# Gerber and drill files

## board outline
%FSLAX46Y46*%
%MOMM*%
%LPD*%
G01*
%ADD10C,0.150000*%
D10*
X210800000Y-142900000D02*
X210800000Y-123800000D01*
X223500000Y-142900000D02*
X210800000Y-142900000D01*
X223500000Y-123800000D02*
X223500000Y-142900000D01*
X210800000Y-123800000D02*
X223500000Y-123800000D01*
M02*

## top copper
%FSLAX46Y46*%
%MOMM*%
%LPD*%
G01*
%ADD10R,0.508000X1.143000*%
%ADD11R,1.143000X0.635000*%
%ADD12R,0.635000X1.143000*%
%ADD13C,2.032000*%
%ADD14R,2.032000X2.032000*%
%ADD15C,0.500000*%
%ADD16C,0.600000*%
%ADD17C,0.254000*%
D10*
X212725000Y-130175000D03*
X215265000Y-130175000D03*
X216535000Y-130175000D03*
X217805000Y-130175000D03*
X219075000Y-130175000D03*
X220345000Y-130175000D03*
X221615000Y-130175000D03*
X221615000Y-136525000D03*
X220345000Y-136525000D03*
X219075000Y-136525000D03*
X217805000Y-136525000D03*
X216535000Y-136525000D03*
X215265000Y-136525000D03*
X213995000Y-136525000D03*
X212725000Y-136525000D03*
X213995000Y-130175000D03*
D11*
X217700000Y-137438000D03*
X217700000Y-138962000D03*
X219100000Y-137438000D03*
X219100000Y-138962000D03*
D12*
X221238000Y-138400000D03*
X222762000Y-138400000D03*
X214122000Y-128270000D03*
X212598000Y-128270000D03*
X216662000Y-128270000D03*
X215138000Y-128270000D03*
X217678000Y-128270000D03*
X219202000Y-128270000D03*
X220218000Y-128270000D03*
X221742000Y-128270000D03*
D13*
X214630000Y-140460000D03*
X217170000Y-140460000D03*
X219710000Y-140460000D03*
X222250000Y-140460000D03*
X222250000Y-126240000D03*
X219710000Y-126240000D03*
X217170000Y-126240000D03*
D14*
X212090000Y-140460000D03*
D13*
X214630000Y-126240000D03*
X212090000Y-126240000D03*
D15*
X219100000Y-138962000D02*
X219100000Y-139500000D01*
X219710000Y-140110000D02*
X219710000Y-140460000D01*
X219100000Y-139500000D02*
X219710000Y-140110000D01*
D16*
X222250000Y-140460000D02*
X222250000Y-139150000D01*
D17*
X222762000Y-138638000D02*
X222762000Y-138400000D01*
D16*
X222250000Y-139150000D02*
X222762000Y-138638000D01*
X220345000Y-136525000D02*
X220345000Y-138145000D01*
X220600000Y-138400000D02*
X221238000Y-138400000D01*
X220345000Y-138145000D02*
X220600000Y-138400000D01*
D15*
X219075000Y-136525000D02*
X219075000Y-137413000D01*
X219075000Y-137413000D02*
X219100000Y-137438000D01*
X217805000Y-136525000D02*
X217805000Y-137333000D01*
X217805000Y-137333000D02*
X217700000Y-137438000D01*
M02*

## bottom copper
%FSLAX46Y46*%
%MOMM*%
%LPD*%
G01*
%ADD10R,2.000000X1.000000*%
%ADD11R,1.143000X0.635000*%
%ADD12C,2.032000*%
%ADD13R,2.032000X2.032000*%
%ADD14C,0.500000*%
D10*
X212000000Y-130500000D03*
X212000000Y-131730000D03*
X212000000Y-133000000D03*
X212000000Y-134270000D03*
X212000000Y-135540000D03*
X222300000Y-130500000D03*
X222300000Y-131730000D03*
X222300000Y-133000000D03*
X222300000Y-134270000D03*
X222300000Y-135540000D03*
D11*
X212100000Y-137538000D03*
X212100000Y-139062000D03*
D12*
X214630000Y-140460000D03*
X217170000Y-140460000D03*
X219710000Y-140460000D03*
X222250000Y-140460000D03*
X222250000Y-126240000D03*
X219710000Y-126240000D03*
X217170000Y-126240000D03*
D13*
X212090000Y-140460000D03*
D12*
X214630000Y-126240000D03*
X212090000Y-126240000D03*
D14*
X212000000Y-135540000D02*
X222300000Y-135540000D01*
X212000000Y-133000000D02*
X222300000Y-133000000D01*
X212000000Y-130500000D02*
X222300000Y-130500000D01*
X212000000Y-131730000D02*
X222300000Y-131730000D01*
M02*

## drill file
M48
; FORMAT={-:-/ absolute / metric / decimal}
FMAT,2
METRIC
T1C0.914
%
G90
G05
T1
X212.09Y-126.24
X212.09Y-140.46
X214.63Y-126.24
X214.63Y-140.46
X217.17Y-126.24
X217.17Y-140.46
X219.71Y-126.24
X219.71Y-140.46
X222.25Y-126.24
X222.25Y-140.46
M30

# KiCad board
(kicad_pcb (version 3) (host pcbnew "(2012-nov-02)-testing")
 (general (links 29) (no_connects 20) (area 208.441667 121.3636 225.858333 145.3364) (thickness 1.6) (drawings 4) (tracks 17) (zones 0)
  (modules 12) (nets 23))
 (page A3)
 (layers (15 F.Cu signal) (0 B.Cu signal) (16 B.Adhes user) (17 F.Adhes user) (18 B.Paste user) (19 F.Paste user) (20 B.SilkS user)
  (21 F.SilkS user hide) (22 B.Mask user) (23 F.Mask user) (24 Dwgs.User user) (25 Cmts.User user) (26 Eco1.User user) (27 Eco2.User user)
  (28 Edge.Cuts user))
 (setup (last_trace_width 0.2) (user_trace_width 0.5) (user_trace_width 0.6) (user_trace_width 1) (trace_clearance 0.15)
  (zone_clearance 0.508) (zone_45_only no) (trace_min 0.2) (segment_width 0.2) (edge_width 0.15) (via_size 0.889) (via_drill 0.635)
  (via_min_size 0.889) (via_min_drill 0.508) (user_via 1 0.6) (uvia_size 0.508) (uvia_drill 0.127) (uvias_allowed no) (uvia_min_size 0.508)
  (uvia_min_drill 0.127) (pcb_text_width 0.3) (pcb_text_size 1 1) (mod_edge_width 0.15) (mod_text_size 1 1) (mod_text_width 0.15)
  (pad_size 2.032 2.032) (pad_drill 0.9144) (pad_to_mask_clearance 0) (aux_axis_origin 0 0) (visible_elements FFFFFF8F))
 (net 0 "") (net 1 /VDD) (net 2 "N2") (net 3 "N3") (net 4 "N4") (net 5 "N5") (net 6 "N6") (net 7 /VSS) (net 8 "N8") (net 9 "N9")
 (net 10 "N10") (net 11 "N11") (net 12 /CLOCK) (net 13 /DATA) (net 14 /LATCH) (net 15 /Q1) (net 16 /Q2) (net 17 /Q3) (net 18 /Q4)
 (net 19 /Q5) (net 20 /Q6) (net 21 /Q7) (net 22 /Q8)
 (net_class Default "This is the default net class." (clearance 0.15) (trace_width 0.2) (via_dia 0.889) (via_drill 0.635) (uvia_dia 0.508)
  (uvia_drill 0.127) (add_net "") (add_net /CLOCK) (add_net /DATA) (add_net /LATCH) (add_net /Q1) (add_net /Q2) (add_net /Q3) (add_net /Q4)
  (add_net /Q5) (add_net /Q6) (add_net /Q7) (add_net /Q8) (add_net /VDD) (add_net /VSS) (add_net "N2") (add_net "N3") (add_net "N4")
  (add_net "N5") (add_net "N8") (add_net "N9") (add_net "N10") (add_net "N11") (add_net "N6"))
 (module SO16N (layer F.Cu) (at 217.17 133.35)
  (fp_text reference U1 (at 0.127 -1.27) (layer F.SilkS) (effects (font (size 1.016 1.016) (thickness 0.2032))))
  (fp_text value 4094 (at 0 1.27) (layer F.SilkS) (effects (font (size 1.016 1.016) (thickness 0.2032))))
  (pad 16 smd rect (at -4.445 -3.175) (size 0.508 1.143) (layers F.Cu F.Paste F.Mask) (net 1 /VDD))
  (pad 14 smd rect (at -1.905 -3.175) (size 0.508 1.143) (layers F.Cu F.Paste F.Mask) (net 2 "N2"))
  (pad 13 smd rect (at -0.635 -3.175) (size 0.508 1.143) (layers F.Cu F.Paste F.Mask) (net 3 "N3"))
  (pad 12 smd rect (at 0.635 -3.175) (size 0.508 1.143) (layers F.Cu F.Paste F.Mask) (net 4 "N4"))
  (pad 11 smd rect (at 1.905 -3.175) (size 0.508 1.143) (layers F.Cu F.Paste F.Mask) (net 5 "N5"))
  (pad 10 smd rect (at 3.175 -3.175) (size 0.508 1.143) (layers F.Cu F.Paste F.Mask) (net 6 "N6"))
  (pad 9 smd rect (at 4.445 -3.175) (size 0.508 1.143) (layers F.Cu F.Paste F.Mask))
  (pad 8 smd rect (at 4.445 3.175) (size 0.508 1.143) (layers F.Cu F.Paste F.Mask) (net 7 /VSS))
  (pad 7 smd rect (at 3.175 3.175) (size 0.508 1.143) (layers F.Cu F.Paste F.Mask) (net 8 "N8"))
  (pad 6 smd rect (at 1.905 3.175) (size 0.508 1.143) (layers F.Cu F.Paste F.Mask) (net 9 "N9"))
  (pad 5 smd rect (at 0.635 3.175) (size 0.508 1.143) (layers F.Cu F.Paste F.Mask) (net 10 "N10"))
  (pad 4 smd rect (at -0.635 3.175) (size 0.508 1.143) (layers F.Cu F.Paste F.Mask) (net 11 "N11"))
  (pad 3 smd rect (at -1.905 3.175) (size 0.508 1.143) (layers F.Cu F.Paste F.Mask) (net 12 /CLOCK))
  (pad 2 smd rect (at -3.175 3.175) (size 0.508 1.143) (layers F.Cu F.Paste F.Mask) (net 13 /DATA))
  (pad 1 smd rect (at -4.445 3.175) (size 0.508 1.143) (layers F.Cu F.Paste F.Mask) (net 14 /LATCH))
  (pad 15 smd rect (at -3.175 -3.175) (size 0.508 1.143) (layers F.Cu F.Paste F.Mask) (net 1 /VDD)))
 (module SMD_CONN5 (layer B.Cu) (at 212 133 180)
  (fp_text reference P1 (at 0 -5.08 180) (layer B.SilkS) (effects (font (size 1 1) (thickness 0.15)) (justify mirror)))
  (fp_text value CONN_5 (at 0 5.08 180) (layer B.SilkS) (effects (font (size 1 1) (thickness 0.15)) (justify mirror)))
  (pad 1 smd rect (at 0 2.5 180) (size 2 1) (layers B.Cu B.Paste B.Mask) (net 1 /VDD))
  (pad 2 smd rect (at 0 1.27 180) (size 2 1) (layers B.Cu B.Paste B.Mask) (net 7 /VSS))
  (pad 3 smd rect (at 0 0 180) (size 2 1) (layers B.Cu B.Paste B.Mask) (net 14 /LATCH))
  (pad 4 smd rect (at 0 -1.27 180) (size 2 1) (layers B.Cu B.Paste B.Mask) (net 13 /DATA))
  (pad 5 smd rect (at 0 -2.54 180) (size 2 1) (layers B.Cu B.Paste B.Mask) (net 12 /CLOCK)))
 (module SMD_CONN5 (layer B.Cu) (at 222.3 133 180)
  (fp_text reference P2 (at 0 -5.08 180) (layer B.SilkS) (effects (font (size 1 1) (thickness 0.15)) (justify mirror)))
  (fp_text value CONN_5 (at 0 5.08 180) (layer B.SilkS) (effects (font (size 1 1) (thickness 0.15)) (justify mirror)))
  (pad 1 smd rect (at 0 2.5 180) (size 2 1) (layers B.Cu B.Paste B.Mask) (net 1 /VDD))
  (pad 2 smd rect (at 0 1.27 180) (size 2 1) (layers B.Cu B.Paste B.Mask) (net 7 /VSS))
  (pad 3 smd rect (at 0 0 180) (size 2 1) (layers B.Cu B.Paste B.Mask) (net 14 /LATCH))
  (pad 4 smd rect (at 0 -1.27 180) (size 2 1) (layers B.Cu B.Paste B.Mask) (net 6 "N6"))
  (pad 5 smd rect (at 0 -2.54 180) (size 2 1) (layers B.Cu B.Paste B.Mask) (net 12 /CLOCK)))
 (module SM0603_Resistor (layer B.Cu) (at 212.1 138.3 270)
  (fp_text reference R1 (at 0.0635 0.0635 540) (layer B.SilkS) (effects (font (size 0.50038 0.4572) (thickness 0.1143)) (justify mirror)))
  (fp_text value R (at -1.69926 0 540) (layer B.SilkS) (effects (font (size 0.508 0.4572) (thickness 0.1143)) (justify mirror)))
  (pad 1 smd rect (at -0.762 0 270) (size 0.635 1.143) (layers B.Cu B.Paste B.Mask) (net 11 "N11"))
  (pad 2 smd rect (at 0.762 0 270) (size 0.635 1.143) (layers B.Cu B.Paste B.Mask) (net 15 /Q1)))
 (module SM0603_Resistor (layer F.Cu) (at 217.7 138.2 270)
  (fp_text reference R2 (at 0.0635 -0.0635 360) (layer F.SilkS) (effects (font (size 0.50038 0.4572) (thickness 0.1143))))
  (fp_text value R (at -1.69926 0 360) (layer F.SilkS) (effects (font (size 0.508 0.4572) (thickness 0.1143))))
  (pad 1 smd rect (at -0.762 0 270) (size 0.635 1.143) (layers F.Cu F.Paste F.Mask) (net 10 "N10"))
  (pad 2 smd rect (at 0.762 0 270) (size 0.635 1.143) (layers F.Cu F.Paste F.Mask) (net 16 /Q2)))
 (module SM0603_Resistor (layer F.Cu) (at 219.1 138.2 270)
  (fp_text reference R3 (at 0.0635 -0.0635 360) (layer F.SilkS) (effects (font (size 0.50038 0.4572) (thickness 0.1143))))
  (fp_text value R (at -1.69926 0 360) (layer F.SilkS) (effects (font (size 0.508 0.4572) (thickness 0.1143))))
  (pad 1 smd rect (at -0.762 0 270) (size 0.635 1.143) (layers F.Cu F.Paste F.Mask) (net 9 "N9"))
  (pad 2 smd rect (at 0.762 0 270) (size 0.635 1.143) (layers F.Cu F.Paste F.Mask) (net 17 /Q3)))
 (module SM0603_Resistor (layer F.Cu) (at 222 138.4)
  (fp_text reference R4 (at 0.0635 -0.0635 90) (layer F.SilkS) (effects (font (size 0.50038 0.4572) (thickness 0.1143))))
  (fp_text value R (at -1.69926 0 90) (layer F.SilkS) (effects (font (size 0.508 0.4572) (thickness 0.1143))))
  (pad 1 smd rect (at -0.762 0) (size 0.635 1.143) (layers F.Cu F.Paste F.Mask) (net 8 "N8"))
  (pad 2 smd rect (at 0.762 0) (size 0.635 1.143) (layers F.Cu F.Paste F.Mask) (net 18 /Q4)))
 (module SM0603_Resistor (layer F.Cu) (at 213.36 128.27 180)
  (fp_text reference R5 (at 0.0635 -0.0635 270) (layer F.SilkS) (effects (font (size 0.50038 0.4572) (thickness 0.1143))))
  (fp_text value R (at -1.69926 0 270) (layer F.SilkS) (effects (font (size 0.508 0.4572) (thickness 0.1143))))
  (pad 1 smd rect (at -0.762 0 180) (size 0.635 1.143) (layers F.Cu F.Paste F.Mask) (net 2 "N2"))
  (pad 2 smd rect (at 0.762 0 180) (size 0.635 1.143) (layers F.Cu F.Paste F.Mask) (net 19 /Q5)))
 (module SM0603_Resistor (layer F.Cu) (at 215.9 128.27 180)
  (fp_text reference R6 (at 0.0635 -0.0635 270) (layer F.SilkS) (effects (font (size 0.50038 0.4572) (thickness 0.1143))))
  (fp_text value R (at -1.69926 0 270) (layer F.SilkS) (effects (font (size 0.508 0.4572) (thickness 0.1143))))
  (pad 1 smd rect (at -0.762 0 180) (size 0.635 1.143) (layers F.Cu F.Paste F.Mask) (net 3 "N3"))
  (pad 2 smd rect (at 0.762 0 180) (size 0.635 1.143) (layers F.Cu F.Paste F.Mask) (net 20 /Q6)))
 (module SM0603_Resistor (layer F.Cu) (at 218.44 128.27)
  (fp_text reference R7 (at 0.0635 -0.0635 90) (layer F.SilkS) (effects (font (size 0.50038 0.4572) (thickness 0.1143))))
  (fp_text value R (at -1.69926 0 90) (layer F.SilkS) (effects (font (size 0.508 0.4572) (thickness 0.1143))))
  (pad 1 smd rect (at -0.762 0) (size 0.635 1.143) (layers F.Cu F.Paste F.Mask) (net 4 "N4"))
  (pad 2 smd rect (at 0.762 0) (size 0.635 1.143) (layers F.Cu F.Paste F.Mask) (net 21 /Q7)))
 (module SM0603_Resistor (layer F.Cu) (at 220.98 128.27)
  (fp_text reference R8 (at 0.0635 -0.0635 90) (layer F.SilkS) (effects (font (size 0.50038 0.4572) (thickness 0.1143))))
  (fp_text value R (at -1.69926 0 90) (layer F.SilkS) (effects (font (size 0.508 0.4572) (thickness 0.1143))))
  (pad 1 smd rect (at -0.762 0) (size 0.635 1.143) (layers F.Cu F.Paste F.Mask) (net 5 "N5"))
  (pad 2 smd rect (at 0.762 0) (size 0.635 1.143) (layers F.Cu F.Paste F.Mask) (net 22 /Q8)))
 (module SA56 (layer F.Cu) (at 217.17 133.35)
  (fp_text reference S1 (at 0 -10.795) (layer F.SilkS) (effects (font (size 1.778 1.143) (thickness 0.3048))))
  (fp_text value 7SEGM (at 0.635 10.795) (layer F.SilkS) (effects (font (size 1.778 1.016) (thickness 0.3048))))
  (pad 2 thru_hole circle (at -2.54 7.11) (size 2.032 2.032) (drill 0.9144) (layers *.Cu *.Mask F.SilkS) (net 16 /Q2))
  (pad 3 thru_hole circle (at 0 7.11) (size 2.032 2.032) (drill 0.9144) (layers *.Cu *.Mask F.SilkS) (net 1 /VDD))
  (pad 4 thru_hole circle (at 2.54 7.11) (size 2.032 2.032) (drill 0.9144) (layers *.Cu *.Mask F.SilkS) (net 17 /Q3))
  (pad 5 thru_hole circle (at 5.08 7.11) (size 2.032 2.032) (drill 0.9144) (layers *.Cu *.Mask F.SilkS) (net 18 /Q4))
  (pad 6 thru_hole circle (at 5.08 -7.11) (size 2.032 2.032) (drill 0.9144) (layers *.Cu *.Mask F.SilkS) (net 22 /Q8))
  (pad 7 thru_hole circle (at 2.54 -7.11) (size 2.032 2.032) (drill 0.9144) (layers *.Cu *.Mask F.SilkS) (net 21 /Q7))
  (pad 8 thru_hole circle (at 0 -7.11) (size 2.032 2.032) (drill 0.9144) (layers *.Cu *.Mask F.SilkS) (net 1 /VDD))
  (pad 1 thru_hole rect (at -5.08 7.11) (size 2.032 2.032) (drill 0.9144) (layers *.Cu *.Mask F.SilkS) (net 15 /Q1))
  (pad 9 thru_hole circle (at -2.54 -7.11) (size 2.032 2.032) (drill 0.9144) (layers *.Cu *.Mask F.SilkS) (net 20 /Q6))
  (pad 10 thru_hole circle (at -5.08 -7.11) (size 2.032 2.032) (drill 0.9144) (layers *.Cu *.Mask F.SilkS) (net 19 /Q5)))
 (gr_line (start 210.8 142.9) (end 210.8 123.8) (angle 90) (layer Edge.Cuts) (width 0.15))
 (gr_line (start 223.5 142.9) (end 210.8 142.9) (angle 90) (layer Edge.Cuts) (width 0.15))
 (gr_line (start 223.5 123.8) (end 223.5 142.9) (angle 90) (layer Edge.Cuts) (width 0.15))
 (gr_line (start 210.8 123.8) (end 223.5 123.8) (angle 90) (layer Edge.Cuts) (width 0.15))
 (segment (start 212 135.54) (end 222.3 135.54) (width 0.5) (layer B.Cu) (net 12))
 (segment (start 212 133) (end 222.3 133) (width 0.5) (layer B.Cu) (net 14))
 (segment (start 219.1 138.962) (end 219.1 139.5) (width 0.5) (layer F.Cu) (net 17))
 (segment (start 219.71 140.11) (end 219.71 140.46) (width 0.5) (layer F.Cu) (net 17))
 (segment (start 219.1 139.5) (end 219.71 140.11) (width 0.5) (layer F.Cu) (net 17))
 (segment (start 222.25 140.46) (end 222.25 139.15) (width 0.6) (layer F.Cu) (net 18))
 (segment (start 222.762 138.638) (end 222.762 138.4) (width 0.254) (layer F.Cu) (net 18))
 (segment (start 222.25 139.15) (end 222.762 138.638) (width 0.6) (layer F.Cu) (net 18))
 (segment (start 212 130.5) (end 222.3 130.5) (width 0.5) (layer B.Cu) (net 1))
 (segment (start 212 131.73) (end 222.3 131.73) (width 0.5) (layer B.Cu) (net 7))
 (segment (start 220.345 136.525) (end 220.345 138.145) (width 0.6) (layer F.Cu) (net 8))
 (segment (start 220.6 138.4) (end 221.238 138.4) (width 0.6) (layer F.Cu) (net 8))
 (segment (start 220.345 138.145) (end 220.6 138.4) (width 0.6) (layer F.Cu) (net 8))
 (segment (start 219.075 136.525) (end 219.075 137.413) (width 0.5) (layer F.Cu) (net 9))
 (segment (start 219.075 137.413) (end 219.1 137.438) (width 0.5) (layer F.Cu) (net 9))
 (segment (start 217.805 136.525) (end 217.805 137.333) (width 0.5) (layer F.Cu) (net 10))
 (segment (start 217.805 137.333) (end 217.7 137.438) (width 0.5) (layer F.Cu) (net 10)))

